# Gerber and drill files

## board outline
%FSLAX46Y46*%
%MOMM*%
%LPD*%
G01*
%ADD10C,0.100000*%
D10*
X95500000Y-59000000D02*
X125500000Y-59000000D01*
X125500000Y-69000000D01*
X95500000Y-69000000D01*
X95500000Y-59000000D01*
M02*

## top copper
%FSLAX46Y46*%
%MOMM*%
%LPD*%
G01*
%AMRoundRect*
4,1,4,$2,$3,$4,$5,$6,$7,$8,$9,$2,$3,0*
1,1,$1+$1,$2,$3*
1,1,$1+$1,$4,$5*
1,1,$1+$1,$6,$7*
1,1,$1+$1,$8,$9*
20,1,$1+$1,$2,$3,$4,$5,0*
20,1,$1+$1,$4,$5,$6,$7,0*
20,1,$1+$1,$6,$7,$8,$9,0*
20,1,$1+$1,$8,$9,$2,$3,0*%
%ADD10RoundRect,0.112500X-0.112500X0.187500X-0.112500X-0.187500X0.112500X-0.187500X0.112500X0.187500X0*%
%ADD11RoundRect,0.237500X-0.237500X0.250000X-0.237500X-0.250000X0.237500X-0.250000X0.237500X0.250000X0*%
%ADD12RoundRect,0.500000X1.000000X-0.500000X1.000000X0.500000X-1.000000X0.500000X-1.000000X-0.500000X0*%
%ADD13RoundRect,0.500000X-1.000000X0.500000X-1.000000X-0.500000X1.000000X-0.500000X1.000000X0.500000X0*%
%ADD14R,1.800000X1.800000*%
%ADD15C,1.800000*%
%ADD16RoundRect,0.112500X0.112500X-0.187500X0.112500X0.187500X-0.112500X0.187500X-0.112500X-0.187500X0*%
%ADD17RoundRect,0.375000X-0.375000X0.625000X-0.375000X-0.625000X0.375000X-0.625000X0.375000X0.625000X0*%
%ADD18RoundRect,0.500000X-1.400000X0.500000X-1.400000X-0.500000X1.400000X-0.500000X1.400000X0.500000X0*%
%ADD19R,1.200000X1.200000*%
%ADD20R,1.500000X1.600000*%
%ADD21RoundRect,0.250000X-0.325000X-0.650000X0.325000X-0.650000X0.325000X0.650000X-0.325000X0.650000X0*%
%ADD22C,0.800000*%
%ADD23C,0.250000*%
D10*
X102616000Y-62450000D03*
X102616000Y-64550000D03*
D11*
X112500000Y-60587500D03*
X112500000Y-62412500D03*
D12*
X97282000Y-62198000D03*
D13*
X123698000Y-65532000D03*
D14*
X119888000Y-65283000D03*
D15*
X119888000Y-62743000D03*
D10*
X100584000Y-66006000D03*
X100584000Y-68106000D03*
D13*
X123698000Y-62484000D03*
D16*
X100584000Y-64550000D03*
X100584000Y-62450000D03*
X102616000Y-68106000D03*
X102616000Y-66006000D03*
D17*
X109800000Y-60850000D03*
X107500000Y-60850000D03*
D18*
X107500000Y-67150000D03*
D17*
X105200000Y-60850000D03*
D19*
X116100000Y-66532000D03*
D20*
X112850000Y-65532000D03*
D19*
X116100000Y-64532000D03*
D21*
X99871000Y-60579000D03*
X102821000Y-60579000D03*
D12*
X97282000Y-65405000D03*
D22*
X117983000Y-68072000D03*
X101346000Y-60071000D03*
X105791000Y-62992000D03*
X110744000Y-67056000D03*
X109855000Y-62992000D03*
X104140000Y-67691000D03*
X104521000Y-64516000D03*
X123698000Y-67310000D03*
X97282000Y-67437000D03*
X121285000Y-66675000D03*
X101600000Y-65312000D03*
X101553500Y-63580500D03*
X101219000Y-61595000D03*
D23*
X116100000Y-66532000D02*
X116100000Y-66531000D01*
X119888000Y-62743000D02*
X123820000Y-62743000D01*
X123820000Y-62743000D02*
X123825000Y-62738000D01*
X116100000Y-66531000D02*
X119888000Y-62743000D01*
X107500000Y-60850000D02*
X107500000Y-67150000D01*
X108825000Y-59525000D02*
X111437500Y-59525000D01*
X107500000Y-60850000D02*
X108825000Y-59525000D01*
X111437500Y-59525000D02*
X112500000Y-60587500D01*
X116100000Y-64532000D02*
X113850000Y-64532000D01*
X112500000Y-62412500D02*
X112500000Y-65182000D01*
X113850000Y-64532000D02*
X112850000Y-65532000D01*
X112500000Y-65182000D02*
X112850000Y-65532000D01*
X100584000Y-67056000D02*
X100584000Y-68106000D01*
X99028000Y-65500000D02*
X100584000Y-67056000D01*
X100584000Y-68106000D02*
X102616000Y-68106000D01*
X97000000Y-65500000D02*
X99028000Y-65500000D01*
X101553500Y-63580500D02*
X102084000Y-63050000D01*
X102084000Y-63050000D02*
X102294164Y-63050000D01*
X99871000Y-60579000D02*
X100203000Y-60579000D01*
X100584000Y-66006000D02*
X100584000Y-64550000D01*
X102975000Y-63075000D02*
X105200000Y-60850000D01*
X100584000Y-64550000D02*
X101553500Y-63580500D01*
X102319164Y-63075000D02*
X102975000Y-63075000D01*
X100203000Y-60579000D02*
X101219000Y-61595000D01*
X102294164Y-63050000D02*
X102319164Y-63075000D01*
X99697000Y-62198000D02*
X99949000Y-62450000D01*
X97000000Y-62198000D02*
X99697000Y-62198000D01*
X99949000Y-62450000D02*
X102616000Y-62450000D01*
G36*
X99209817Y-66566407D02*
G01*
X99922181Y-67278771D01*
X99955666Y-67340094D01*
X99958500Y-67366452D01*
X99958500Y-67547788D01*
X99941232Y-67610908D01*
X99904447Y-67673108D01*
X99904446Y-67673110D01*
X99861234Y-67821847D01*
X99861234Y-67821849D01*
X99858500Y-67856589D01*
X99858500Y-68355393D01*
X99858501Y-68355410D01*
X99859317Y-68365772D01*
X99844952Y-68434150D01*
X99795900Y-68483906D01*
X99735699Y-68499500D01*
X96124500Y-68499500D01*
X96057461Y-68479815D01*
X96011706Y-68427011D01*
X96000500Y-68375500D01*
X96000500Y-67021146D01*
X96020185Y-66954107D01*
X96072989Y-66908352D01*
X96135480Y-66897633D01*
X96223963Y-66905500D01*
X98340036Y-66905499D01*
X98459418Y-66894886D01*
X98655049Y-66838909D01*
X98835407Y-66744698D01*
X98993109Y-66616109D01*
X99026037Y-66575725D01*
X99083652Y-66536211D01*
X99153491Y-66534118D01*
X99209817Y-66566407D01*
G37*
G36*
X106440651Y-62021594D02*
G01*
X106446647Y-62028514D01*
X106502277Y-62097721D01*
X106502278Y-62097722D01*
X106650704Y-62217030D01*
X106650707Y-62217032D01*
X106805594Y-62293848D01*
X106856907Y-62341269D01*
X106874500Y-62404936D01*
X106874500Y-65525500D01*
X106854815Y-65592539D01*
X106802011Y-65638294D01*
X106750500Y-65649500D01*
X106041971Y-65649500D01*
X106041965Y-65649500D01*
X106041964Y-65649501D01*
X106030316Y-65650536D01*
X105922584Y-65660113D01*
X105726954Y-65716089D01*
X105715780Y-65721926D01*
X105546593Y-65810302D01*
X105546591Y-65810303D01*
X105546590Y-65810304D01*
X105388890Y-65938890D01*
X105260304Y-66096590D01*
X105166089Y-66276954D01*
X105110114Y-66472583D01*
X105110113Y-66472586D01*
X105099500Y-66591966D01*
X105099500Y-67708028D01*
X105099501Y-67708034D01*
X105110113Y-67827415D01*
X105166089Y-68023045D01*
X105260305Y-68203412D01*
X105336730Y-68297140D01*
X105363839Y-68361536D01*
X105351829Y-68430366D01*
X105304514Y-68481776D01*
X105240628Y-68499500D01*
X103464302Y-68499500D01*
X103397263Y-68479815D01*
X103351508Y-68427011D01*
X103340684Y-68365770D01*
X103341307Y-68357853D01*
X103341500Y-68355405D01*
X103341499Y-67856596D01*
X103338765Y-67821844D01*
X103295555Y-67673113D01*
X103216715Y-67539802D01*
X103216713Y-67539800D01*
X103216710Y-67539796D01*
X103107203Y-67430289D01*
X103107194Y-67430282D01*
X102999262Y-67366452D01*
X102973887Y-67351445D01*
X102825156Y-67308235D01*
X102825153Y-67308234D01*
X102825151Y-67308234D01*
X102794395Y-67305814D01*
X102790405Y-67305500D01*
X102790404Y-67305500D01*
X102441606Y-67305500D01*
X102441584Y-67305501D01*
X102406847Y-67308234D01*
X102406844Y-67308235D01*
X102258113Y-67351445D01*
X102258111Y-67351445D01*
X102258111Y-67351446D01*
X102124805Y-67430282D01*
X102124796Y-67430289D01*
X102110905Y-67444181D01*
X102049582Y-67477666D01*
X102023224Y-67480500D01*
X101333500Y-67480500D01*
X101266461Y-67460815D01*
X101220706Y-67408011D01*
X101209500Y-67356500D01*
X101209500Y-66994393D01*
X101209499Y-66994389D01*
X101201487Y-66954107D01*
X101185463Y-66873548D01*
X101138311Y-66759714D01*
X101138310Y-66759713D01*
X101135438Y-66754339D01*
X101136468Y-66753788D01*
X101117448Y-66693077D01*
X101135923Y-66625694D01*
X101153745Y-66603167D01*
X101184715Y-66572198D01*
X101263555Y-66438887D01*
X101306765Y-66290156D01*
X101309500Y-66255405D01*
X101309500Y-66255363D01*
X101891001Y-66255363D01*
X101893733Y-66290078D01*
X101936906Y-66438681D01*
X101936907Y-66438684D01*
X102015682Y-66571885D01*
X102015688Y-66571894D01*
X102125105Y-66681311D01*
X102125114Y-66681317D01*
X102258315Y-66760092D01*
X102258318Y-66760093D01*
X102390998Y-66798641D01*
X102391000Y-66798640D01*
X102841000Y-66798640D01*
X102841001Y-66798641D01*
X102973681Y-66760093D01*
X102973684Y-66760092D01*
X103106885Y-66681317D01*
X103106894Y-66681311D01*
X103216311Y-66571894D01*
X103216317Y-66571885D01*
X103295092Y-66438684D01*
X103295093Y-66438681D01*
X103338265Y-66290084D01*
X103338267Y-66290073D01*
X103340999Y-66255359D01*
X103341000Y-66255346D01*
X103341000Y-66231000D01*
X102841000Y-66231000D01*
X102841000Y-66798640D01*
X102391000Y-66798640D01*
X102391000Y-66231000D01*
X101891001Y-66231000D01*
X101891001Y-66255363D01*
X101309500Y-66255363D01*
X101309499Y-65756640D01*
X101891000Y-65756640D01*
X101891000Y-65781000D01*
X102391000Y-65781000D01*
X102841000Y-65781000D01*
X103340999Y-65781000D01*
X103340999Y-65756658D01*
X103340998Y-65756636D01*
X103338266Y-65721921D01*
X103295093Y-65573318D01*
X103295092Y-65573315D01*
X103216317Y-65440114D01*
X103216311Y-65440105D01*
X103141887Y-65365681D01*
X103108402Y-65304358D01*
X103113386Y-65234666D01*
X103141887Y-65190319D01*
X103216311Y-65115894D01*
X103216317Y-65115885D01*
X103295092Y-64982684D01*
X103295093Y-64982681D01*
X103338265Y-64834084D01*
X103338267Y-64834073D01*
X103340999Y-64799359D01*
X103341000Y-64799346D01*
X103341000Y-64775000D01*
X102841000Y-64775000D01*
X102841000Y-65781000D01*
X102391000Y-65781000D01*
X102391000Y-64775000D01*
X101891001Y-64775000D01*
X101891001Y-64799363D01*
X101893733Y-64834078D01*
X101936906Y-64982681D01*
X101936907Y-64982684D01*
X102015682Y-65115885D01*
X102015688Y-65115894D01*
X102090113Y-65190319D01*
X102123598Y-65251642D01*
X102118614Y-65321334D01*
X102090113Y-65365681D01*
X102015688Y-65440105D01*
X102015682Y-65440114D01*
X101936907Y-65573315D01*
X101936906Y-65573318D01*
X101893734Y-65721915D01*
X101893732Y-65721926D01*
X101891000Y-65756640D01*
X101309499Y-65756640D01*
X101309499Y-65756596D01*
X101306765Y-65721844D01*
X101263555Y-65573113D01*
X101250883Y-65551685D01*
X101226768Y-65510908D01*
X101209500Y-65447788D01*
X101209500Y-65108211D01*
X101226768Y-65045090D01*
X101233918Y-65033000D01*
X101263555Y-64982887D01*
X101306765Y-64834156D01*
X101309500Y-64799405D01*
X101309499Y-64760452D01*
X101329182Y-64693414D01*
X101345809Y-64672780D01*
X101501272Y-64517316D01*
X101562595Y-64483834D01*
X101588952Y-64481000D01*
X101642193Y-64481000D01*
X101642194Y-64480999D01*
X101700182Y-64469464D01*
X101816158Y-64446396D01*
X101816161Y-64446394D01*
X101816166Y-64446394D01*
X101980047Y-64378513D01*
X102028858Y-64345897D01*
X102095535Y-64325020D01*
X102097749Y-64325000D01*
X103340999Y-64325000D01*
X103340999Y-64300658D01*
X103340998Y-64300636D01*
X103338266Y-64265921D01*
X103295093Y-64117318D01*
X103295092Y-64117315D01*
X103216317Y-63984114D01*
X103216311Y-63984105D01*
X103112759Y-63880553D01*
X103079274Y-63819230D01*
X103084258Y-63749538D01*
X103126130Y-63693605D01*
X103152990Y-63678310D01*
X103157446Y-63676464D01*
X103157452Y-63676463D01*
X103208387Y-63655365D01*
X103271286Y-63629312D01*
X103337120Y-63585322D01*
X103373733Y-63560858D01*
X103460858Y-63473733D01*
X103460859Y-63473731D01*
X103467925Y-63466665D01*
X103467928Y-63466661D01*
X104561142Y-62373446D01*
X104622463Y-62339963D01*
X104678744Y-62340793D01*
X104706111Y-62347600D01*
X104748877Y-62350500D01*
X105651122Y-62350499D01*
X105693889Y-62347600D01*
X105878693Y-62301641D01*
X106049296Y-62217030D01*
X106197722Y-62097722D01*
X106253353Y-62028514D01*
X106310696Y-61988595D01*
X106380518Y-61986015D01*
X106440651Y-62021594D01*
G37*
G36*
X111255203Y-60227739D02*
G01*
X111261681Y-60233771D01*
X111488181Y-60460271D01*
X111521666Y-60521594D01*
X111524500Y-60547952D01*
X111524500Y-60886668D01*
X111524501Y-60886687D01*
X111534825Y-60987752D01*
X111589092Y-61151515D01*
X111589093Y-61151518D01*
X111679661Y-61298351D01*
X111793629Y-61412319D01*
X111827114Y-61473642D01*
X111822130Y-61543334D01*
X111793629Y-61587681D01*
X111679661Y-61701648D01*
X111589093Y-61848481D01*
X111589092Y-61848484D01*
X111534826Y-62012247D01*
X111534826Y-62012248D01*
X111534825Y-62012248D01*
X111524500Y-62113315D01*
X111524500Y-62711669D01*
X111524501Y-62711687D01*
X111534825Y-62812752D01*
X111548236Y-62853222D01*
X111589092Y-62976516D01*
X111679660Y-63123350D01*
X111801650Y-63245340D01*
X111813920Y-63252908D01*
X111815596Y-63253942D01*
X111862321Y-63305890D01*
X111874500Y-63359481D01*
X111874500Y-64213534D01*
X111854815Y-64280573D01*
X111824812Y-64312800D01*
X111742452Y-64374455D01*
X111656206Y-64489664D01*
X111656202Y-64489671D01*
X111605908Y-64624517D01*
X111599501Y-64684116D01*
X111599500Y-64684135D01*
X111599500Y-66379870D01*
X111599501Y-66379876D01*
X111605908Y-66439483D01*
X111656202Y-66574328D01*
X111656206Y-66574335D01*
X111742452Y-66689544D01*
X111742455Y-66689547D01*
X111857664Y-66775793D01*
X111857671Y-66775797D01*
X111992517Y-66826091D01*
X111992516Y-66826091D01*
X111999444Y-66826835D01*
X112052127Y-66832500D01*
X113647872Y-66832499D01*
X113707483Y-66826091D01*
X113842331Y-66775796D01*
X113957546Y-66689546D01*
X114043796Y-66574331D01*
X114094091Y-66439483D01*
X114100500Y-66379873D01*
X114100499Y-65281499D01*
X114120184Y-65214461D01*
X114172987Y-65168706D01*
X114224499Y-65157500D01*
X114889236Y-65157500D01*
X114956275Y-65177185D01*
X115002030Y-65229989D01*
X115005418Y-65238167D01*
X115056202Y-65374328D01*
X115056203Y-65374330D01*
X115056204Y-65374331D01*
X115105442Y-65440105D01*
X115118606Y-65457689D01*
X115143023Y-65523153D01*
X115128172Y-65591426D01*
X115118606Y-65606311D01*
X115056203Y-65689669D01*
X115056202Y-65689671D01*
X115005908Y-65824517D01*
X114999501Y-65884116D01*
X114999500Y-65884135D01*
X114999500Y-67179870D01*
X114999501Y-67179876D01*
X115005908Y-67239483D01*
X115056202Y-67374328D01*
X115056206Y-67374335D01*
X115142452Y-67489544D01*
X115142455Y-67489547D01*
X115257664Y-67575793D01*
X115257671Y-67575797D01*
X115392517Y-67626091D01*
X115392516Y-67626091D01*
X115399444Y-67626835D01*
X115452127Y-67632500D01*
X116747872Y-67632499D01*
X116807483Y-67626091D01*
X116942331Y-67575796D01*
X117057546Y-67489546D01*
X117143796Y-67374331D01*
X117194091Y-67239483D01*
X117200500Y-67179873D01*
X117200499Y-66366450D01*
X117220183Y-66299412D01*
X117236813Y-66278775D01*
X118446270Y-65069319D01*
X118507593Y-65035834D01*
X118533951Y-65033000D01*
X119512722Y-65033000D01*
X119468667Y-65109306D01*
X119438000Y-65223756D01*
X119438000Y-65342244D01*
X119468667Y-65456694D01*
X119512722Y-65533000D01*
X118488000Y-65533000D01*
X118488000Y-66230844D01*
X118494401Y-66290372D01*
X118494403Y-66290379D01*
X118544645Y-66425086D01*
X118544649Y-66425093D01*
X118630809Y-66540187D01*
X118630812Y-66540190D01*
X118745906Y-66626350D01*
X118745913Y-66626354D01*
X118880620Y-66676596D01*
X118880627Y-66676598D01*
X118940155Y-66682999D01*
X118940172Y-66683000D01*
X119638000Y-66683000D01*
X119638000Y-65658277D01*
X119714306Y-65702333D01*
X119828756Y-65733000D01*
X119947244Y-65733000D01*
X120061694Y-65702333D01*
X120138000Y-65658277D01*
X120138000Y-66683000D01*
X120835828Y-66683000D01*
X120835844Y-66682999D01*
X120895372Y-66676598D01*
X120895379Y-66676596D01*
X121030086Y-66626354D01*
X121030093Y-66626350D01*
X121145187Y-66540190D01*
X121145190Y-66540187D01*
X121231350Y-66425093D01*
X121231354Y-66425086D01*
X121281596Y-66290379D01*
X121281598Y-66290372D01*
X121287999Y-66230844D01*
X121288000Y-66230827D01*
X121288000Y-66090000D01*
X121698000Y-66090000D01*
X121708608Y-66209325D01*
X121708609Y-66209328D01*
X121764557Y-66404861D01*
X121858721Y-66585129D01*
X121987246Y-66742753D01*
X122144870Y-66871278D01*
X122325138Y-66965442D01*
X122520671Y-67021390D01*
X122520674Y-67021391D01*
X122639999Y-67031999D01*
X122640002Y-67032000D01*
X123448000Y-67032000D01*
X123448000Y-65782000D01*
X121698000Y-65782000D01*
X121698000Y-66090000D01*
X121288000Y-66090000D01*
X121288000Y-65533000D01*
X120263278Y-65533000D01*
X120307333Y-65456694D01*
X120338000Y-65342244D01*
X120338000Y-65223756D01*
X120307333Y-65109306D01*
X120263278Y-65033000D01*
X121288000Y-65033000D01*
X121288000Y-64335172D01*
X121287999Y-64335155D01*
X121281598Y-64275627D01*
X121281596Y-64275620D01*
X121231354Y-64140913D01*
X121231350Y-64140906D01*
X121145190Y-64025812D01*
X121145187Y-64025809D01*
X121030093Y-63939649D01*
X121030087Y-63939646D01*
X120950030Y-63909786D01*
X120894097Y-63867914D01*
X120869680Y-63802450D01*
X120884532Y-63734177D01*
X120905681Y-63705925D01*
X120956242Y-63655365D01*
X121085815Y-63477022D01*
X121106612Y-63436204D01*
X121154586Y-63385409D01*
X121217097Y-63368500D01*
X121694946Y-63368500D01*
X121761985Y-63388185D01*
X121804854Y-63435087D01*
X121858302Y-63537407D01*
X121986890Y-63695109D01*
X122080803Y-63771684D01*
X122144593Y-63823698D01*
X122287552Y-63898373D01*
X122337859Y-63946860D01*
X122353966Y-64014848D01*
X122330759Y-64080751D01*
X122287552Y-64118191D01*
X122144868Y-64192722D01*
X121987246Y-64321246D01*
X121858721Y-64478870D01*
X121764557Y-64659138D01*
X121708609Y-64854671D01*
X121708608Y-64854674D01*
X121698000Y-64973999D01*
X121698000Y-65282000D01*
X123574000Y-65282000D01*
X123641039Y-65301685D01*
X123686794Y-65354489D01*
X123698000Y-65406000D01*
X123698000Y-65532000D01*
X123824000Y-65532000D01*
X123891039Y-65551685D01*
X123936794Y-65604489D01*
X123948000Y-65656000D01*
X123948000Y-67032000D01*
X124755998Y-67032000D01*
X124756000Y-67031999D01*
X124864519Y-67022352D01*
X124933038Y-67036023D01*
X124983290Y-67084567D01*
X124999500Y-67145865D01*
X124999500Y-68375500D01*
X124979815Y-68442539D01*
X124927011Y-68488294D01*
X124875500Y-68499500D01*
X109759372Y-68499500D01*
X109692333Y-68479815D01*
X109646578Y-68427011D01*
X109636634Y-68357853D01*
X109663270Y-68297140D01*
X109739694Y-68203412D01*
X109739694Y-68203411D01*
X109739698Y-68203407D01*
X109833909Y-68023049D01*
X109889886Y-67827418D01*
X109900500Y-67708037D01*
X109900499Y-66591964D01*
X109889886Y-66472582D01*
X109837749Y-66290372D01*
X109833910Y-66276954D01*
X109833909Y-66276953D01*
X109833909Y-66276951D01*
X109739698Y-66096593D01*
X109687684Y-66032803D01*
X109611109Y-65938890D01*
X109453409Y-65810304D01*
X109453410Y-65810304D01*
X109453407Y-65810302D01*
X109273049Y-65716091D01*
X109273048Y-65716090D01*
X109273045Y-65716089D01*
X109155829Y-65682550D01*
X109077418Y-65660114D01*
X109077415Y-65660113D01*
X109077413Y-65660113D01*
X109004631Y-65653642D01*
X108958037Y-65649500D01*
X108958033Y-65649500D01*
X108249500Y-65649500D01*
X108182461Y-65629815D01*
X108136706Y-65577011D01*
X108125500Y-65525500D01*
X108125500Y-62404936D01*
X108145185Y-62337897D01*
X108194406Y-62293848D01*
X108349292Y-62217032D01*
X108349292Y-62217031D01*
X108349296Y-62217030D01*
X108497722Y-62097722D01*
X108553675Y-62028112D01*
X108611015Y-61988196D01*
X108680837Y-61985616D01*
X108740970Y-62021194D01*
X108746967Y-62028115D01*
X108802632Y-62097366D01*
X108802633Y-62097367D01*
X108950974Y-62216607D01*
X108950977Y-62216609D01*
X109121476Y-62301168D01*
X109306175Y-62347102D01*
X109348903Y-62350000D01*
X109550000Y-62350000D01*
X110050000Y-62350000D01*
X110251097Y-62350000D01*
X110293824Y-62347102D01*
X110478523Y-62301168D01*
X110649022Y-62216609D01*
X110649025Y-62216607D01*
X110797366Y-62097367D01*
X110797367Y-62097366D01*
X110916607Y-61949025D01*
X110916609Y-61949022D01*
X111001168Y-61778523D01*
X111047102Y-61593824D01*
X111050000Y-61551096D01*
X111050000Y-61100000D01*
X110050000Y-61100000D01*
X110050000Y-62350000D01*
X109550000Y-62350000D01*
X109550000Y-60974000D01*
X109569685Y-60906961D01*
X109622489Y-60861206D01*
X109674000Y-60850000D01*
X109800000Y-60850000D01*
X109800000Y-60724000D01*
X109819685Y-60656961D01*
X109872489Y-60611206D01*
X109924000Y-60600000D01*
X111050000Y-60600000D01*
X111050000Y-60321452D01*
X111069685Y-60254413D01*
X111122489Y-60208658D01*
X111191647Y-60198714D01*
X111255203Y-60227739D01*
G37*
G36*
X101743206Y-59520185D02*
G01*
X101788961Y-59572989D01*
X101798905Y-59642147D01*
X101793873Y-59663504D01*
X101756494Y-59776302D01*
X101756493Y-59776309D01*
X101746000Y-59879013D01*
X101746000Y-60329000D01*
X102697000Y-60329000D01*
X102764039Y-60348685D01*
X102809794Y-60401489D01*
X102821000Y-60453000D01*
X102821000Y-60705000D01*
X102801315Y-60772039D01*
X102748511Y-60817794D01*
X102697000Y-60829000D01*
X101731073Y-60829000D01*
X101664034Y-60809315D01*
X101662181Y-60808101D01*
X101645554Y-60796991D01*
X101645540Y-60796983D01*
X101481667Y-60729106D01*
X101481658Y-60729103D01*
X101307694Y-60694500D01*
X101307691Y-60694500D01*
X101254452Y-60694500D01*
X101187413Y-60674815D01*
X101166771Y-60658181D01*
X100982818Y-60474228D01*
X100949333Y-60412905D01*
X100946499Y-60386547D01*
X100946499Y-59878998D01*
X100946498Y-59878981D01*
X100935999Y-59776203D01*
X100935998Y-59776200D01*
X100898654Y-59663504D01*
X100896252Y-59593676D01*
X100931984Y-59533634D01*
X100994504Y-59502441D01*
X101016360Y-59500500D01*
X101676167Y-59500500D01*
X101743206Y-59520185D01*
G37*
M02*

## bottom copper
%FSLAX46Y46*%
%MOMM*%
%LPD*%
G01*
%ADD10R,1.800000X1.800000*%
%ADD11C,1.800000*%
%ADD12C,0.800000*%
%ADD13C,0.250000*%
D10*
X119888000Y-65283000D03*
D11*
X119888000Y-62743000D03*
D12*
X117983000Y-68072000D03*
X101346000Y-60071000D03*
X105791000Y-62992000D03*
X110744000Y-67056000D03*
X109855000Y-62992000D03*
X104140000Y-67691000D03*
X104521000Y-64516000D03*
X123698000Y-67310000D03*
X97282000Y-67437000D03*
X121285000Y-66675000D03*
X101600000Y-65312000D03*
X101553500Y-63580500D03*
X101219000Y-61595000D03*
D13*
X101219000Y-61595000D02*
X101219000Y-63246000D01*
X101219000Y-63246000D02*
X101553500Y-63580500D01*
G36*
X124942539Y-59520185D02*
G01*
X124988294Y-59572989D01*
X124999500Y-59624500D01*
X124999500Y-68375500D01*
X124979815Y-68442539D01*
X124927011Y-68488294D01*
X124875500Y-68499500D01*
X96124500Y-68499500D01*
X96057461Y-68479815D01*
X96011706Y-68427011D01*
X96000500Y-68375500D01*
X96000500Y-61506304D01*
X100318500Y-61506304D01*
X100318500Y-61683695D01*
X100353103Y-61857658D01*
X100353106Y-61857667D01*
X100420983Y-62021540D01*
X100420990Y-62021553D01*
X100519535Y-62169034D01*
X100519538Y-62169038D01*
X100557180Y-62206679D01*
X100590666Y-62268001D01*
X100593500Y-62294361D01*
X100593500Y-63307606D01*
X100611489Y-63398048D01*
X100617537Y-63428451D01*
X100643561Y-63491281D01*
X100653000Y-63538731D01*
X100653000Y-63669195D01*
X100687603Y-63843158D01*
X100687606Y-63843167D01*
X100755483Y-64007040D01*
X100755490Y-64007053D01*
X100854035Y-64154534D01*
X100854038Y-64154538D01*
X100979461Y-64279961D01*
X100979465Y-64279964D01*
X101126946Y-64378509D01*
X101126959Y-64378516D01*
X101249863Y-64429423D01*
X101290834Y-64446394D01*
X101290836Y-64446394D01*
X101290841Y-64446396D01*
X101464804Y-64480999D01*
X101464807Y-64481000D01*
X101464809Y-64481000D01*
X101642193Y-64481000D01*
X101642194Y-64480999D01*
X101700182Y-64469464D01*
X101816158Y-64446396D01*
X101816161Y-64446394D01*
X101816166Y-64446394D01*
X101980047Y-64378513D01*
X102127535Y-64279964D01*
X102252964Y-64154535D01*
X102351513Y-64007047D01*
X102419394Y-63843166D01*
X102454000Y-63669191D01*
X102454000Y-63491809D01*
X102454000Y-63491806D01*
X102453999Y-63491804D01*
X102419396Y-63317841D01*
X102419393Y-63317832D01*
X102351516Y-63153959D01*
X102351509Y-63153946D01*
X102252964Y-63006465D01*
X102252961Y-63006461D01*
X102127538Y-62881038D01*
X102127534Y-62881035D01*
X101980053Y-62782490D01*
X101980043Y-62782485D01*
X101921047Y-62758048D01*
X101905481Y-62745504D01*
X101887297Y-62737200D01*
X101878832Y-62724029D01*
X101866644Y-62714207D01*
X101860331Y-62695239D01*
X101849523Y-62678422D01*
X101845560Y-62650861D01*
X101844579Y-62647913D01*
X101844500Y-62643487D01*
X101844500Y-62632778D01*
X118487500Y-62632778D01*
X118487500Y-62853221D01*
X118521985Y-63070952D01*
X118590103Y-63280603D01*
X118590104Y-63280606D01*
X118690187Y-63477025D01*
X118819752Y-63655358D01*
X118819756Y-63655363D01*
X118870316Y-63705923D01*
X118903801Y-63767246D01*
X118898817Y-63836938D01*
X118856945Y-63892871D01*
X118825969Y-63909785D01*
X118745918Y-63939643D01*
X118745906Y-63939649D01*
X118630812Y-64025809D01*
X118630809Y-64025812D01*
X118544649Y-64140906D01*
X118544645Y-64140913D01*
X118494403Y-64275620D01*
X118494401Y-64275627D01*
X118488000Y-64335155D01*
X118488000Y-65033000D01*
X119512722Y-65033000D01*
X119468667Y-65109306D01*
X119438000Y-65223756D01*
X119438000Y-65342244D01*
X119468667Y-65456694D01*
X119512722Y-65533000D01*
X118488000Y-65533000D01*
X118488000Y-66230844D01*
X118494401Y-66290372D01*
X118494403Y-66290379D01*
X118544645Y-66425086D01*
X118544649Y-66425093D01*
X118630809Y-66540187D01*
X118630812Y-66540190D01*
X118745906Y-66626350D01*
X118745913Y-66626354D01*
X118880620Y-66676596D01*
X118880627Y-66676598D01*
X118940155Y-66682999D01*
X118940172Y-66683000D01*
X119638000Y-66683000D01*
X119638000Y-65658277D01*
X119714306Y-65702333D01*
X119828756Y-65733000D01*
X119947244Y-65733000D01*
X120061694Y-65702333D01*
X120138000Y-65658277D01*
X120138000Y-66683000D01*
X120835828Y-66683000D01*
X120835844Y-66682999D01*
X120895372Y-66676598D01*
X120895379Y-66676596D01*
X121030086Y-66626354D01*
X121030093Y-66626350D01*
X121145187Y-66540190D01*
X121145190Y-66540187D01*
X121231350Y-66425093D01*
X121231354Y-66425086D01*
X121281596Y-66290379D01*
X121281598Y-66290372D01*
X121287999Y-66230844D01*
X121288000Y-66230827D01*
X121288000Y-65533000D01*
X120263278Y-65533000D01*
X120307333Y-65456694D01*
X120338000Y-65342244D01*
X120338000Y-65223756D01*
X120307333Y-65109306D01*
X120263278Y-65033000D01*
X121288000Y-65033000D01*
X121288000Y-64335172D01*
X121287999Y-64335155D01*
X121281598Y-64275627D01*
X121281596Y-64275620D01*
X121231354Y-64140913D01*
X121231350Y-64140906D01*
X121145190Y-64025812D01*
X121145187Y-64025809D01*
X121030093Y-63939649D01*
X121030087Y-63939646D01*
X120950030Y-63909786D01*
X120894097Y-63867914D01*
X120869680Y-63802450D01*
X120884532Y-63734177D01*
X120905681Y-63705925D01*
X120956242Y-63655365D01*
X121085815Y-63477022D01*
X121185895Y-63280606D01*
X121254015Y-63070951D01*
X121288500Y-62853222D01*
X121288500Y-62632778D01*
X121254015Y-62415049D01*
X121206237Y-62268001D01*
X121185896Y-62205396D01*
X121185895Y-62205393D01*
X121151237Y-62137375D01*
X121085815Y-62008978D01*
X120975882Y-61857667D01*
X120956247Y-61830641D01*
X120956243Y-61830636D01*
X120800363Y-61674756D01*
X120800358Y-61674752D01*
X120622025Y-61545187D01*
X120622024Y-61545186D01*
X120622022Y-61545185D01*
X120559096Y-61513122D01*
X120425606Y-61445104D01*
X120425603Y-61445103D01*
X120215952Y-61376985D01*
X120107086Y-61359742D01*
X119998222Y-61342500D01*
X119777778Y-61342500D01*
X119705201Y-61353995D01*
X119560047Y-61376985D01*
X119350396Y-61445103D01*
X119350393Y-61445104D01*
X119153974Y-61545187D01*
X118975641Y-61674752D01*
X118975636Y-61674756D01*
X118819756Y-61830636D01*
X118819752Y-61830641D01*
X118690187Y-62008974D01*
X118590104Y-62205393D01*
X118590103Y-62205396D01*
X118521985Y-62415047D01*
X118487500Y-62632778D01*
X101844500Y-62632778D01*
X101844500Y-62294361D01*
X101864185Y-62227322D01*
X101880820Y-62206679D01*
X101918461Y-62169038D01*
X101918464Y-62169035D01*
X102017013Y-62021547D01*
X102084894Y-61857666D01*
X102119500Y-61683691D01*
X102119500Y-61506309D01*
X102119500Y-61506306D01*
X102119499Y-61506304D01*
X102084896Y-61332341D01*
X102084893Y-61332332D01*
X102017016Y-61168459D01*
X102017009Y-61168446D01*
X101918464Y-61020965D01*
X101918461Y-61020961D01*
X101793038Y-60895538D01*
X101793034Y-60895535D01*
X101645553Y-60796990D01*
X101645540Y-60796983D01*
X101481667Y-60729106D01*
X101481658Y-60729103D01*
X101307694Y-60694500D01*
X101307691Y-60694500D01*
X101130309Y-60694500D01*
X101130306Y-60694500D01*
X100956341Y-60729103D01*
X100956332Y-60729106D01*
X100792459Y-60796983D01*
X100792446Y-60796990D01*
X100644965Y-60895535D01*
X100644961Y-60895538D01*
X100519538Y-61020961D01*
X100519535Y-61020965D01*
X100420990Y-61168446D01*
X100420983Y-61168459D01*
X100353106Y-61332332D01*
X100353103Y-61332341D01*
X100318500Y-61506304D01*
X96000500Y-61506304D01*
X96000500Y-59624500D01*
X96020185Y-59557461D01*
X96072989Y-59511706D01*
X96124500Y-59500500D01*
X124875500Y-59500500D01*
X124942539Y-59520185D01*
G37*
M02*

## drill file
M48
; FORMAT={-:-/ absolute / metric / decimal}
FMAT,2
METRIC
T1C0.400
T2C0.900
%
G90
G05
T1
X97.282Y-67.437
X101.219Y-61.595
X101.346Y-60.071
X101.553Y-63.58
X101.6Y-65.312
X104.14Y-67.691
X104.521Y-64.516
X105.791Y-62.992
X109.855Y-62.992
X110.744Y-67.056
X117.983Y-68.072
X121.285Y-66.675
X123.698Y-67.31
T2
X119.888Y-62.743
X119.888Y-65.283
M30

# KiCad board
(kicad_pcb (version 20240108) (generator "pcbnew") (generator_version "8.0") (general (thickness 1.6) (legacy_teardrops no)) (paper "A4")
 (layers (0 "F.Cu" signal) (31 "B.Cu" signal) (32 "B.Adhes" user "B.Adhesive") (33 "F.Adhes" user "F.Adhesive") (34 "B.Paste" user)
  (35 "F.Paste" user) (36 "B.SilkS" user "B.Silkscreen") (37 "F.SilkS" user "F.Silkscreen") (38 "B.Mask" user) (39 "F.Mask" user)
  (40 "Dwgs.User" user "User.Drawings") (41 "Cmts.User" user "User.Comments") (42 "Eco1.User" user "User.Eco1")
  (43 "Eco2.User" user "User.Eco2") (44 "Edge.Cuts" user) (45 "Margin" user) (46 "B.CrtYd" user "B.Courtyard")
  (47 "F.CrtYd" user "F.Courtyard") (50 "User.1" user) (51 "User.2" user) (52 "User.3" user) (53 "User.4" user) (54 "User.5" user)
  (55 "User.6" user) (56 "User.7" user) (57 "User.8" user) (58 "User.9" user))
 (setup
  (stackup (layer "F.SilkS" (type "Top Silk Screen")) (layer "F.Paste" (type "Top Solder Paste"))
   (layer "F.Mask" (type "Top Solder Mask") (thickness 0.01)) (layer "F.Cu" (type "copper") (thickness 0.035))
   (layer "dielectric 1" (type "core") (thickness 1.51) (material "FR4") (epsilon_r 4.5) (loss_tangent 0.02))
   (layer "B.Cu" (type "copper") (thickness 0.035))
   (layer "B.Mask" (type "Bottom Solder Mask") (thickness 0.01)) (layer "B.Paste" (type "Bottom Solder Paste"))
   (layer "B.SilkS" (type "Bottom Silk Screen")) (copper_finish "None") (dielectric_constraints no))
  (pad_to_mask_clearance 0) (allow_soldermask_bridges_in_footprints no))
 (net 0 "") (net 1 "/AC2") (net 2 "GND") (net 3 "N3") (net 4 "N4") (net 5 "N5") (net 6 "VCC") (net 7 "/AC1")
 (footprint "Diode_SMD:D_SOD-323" (layer "F.Cu") (at 102.616 63.5 -90)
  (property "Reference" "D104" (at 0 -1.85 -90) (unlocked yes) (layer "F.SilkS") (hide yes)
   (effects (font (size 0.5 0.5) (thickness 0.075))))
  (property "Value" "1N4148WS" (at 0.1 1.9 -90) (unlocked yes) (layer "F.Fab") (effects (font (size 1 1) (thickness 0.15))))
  (pad "1" smd roundrect (at -1.05 0 270) (size 0.6 0.45) (layers "F.Cu" "F.Paste" "F.Mask") (roundrect_rratio 0.25) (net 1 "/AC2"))
  (pad "2" smd roundrect (at 1.05 0 270) (size 0.6 0.45) (layers "F.Cu" "F.Paste" "F.Mask") (roundrect_rratio 0.25) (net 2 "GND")))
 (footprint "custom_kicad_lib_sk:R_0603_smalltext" (layer "F.Cu") (at 112.5 61.5 -90)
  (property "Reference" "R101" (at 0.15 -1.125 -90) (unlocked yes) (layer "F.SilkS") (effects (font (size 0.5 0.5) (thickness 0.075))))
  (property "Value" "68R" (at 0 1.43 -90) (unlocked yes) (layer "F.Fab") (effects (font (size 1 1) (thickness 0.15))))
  (pad "1" smd roundrect (at -0.9125 0 270) (size 0.975 0.95) (layers "F.Cu" "F.Paste" "F.Mask") (roundrect_rratio 0.25) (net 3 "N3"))
  (pad "2" smd roundrect (at 0.9125 0 270) (size 0.975 0.95) (layers "F.Cu" "F.Paste" "F.Mask") (roundrect_rratio 0.25) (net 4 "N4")))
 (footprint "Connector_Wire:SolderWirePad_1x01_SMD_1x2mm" (layer "F.Cu") (at 97.282 62.198 90)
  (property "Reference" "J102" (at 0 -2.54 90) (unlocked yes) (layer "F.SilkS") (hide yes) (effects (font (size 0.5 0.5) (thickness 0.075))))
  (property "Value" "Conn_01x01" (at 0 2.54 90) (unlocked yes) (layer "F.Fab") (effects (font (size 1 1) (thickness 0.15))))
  (pad "1" smd roundrect (at 0 0 90) (size 2 3) (layers "F.Cu" "F.Paste" "F.Mask") (roundrect_rratio 0.25) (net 1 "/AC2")))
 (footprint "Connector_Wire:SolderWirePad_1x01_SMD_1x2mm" (layer "F.Cu") (at 123.698 65.532 -90)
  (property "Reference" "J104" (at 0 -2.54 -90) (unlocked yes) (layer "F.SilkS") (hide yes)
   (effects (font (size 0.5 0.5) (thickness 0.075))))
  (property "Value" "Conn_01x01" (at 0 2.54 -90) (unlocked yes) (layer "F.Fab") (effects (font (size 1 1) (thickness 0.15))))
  (pad "1" smd roundrect (at 0 0 270) (size 2 3) (layers "F.Cu" "F.Paste" "F.Mask") (roundrect_rratio 0.25) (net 2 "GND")))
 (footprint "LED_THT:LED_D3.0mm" (layer "F.Cu") (at 119.888 65.283 90)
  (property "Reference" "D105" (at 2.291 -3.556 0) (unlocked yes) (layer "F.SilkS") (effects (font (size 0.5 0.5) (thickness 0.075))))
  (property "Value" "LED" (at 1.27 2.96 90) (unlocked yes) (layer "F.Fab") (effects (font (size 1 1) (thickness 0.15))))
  (pad "1" thru_hole rect (at 0 0 90) (size 1.8 1.8) (drill 0.9) (layers "*.Cu" "*.Mask") (remove_unused_layers no) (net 2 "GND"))
  (pad "2" thru_hole circle (at 2.54 0 90) (size 1.8 1.8) (drill 0.9) (layers "*.Cu" "*.Mask") (remove_unused_layers no) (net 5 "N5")))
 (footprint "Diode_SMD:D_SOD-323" (layer "F.Cu") (at 100.584 67.056 -90)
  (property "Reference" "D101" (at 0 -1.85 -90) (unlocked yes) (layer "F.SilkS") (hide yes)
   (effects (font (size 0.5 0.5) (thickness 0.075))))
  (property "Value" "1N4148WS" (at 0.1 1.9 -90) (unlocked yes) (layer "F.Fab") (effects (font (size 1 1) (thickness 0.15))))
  (pad "1" smd roundrect (at -1.05 0 270) (size 0.6 0.45) (layers "F.Cu" "F.Paste" "F.Mask") (roundrect_rratio 0.25) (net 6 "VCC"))
  (pad "2" smd roundrect (at 1.05 0 270) (size 0.6 0.45) (layers "F.Cu" "F.Paste" "F.Mask") (roundrect_rratio 0.25) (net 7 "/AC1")))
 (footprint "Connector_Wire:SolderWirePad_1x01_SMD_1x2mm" (layer "F.Cu") (at 123.698 62.484 -90)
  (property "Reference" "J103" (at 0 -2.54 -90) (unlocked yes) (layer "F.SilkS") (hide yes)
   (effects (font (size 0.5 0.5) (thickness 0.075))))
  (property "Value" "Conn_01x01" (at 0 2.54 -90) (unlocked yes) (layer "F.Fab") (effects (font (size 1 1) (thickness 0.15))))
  (pad "1" smd roundrect (at 0 0 270) (size 2 3) (layers "F.Cu" "F.Paste" "F.Mask") (roundrect_rratio 0.25) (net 5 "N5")))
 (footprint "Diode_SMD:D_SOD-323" (layer "F.Cu") (at 100.584 63.5 90)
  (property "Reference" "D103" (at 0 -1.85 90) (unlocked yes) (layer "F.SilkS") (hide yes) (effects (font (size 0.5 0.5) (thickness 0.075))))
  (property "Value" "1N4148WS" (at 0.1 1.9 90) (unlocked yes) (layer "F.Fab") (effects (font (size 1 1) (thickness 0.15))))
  (pad "1" smd roundrect (at -1.05 0 90) (size 0.6 0.45) (layers "F.Cu" "F.Paste" "F.Mask") (roundrect_rratio 0.25) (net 6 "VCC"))
  (pad "2" smd roundrect (at 1.05 0 90) (size 0.6 0.45) (layers "F.Cu" "F.Paste" "F.Mask") (roundrect_rratio 0.25) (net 1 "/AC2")))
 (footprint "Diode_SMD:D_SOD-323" (layer "F.Cu") (at 102.616 67.056 90)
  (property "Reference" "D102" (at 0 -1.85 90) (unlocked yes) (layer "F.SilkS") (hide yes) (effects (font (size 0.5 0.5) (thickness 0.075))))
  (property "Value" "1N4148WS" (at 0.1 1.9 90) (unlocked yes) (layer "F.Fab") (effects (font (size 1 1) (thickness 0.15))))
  (pad "1" smd roundrect (at -1.05 0 90) (size 0.6 0.45) (layers "F.Cu" "F.Paste" "F.Mask") (roundrect_rratio 0.25) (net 7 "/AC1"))
  (pad "2" smd roundrect (at 1.05 0 90) (size 0.6 0.45) (layers "F.Cu" "F.Paste" "F.Mask") (roundrect_rratio 0.25) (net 2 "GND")))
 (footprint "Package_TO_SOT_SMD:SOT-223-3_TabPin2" (layer "F.Cu") (at 107.5 64 -90)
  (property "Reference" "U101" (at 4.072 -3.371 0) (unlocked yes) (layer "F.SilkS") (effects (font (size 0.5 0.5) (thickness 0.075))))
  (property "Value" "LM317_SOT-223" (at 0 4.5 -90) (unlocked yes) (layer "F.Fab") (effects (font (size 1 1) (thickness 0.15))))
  (pad "1" smd roundrect (at -3.15 -2.3 270) (size 2 1.5) (layers "F.Cu" "F.Paste" "F.Mask") (roundrect_rratio 0.25) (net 2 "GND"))
  (pad "2" smd roundrect (at -3.15 0 270) (size 2 1.5) (layers "F.Cu" "F.Paste" "F.Mask") (roundrect_rratio 0.25) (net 3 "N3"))
  (pad "2" smd roundrect (at 3.15 0 270) (size 2 3.8) (layers "F.Cu" "F.Paste" "F.Mask") (roundrect_rratio 0.25) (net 3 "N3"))
  (pad "3" smd roundrect (at -3.15 2.3 270) (size 2 1.5) (layers "F.Cu" "F.Paste" "F.Mask") (roundrect_rratio 0.25) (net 6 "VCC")))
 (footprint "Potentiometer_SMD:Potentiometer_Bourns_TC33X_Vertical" (layer "F.Cu") (at 114.3 65.532 180)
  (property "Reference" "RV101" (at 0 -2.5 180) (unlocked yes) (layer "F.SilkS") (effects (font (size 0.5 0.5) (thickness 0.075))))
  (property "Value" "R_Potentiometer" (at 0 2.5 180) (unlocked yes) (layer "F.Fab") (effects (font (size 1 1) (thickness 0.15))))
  (pad "1" smd rect (at -1.8 -1 180) (size 1.2 1.2) (layers "F.Cu" "F.Paste" "F.Mask") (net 5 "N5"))
  (pad "2" smd rect (at 1.45 0 180) (size 1.5 1.6) (layers "F.Cu" "F.Paste" "F.Mask") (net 4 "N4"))
  (pad "3" smd rect (at -1.8 1 180) (size 1.2 1.2) (layers "F.Cu" "F.Paste" "F.Mask") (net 4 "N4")))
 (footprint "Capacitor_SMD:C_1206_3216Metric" (layer "F.Cu") (at 101.346 60.579)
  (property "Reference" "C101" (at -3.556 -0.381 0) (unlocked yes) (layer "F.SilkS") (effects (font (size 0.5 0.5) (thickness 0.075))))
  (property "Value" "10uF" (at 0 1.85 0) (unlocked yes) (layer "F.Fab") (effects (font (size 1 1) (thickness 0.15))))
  (pad "1" smd roundrect (at -1.475 0) (size 1.15 1.8) (layers "F.Cu" "F.Paste" "F.Mask") (roundrect_rratio 0.217391) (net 6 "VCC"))
  (pad "2" smd roundrect (at 1.475 0) (size 1.15 1.8) (layers "F.Cu" "F.Paste" "F.Mask") (roundrect_rratio 0.217391) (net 2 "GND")))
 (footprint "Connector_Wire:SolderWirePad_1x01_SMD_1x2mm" (layer "F.Cu") (at 97.282 65.405 90)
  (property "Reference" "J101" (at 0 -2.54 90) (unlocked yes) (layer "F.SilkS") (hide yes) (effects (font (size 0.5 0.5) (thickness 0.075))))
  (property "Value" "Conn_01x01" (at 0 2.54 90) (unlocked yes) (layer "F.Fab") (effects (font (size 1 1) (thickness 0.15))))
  (pad "1" smd roundrect (at 0 0 90) (size 2 3) (layers "F.Cu" "F.Paste" "F.Mask") (roundrect_rratio 0.25) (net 7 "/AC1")))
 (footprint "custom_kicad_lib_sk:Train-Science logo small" (layer "B.Cu") (at 101.6 64.008 90)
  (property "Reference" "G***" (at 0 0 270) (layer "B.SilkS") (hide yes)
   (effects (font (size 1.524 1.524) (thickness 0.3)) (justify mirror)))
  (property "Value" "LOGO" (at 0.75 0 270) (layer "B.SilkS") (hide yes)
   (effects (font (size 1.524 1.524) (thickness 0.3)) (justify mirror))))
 (gr_rect (start 95.5 59) (end 125.5 69) (stroke (width 0.1) (type default)) (fill none) (layer "Edge.Cuts"))
 (via (at 117.983 68.072) (size 0.8) (drill 0.4) (layers "F.Cu" "B.Cu") (free yes) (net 2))
 (via (at 101.346 60.071) (size 0.8) (drill 0.4) (layers "F.Cu" "B.Cu") (free yes) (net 2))
 (via (at 105.791 62.992) (size 0.8) (drill 0.4) (layers "F.Cu" "B.Cu") (free yes) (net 2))
 (via (at 110.744 67.056) (size 0.8) (drill 0.4) (layers "F.Cu" "B.Cu") (free yes) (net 2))
 (via (at 109.855 62.992) (size 0.8) (drill 0.4) (layers "F.Cu" "B.Cu") (free yes) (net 2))
 (via (at 104.14 67.691) (size 0.8) (drill 0.4) (layers "F.Cu" "B.Cu") (free yes) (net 2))
 (via (at 104.521 64.516) (size 0.8) (drill 0.4) (layers "F.Cu" "B.Cu") (free yes) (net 2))
 (via (at 123.698 67.31) (size 0.8) (drill 0.4) (layers "F.Cu" "B.Cu") (free yes) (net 2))
 (via (at 97.282 67.437) (size 0.8) (drill 0.4) (layers "F.Cu" "B.Cu") (free yes) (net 2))
 (via (at 121.285 66.675) (size 0.8) (drill 0.4) (layers "F.Cu" "B.Cu") (free yes) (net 2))
 (via (at 101.6 65.312) (size 0.8) (drill 0.4) (layers "F.Cu" "B.Cu") (free yes) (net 2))
 (segment (start 116.1 66.532) (end 116.1 66.531) (width 0.25) (layer "F.Cu") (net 5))
 (segment (start 119.888 62.743) (end 123.82 62.743) (width 0.25) (layer "F.Cu") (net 5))
 (segment (start 123.82 62.743) (end 123.825 62.738) (width 0.25) (layer "F.Cu") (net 5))
 (segment (start 116.1 66.531) (end 119.888 62.743) (width 0.25) (layer "F.Cu") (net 5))
 (segment (start 107.5 60.85) (end 107.5 67.15) (width 0.25) (layer "F.Cu") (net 3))
 (segment (start 108.825 59.525) (end 111.4375 59.525) (width 0.25) (layer "F.Cu") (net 3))
 (segment (start 107.5 60.85) (end 108.825 59.525) (width 0.25) (layer "F.Cu") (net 3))
 (segment (start 111.4375 59.525) (end 112.5 60.5875) (width 0.25) (layer "F.Cu") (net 3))
 (segment (start 116.1 64.532) (end 113.85 64.532) (width 0.25) (layer "F.Cu") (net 4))
 (segment (start 112.5 62.4125) (end 112.5 65.182) (width 0.25) (layer "F.Cu") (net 4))
 (segment (start 113.85 64.532) (end 112.85 65.532) (width 0.25) (layer "F.Cu") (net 4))
 (segment (start 112.5 65.182) (end 112.85 65.532) (width 0.25) (layer "F.Cu") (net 4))
 (segment (start 100.584 67.056) (end 100.584 68.106) (width 0.25) (layer "F.Cu") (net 7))
 (segment (start 99.028 65.5) (end 100.584 67.056) (width 0.25) (layer "F.Cu") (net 7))
 (segment (start 100.584 68.106) (end 102.616 68.106) (width 0.25) (layer "F.Cu") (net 7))
 (segment (start 97 65.5) (end 99.028 65.5) (width 0.25) (layer "F.Cu") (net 7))
 (segment (start 101.5535 63.5805) (end 102.084 63.05) (width 0.25) (layer "F.Cu") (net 6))
 (segment (start 102.084 63.05) (end 102.294164 63.05) (width 0.25) (layer "F.Cu") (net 6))
 (segment (start 99.871 60.579) (end 100.203 60.579) (width 0.25) (layer "F.Cu") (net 6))
 (segment (start 100.584 66.006) (end 100.584 64.55) (width 0.25) (layer "F.Cu") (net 6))
 (segment (start 102.975 63.075) (end 105.2 60.85) (width 0.25) (layer "F.Cu") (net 6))
 (segment (start 100.584 64.55) (end 101.5535 63.5805) (width 0.25) (layer "F.Cu") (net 6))
 (segment (start 102.319164 63.075) (end 102.975 63.075) (width 0.25) (layer "F.Cu") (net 6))
 (segment (start 100.203 60.579) (end 101.219 61.595) (width 0.25) (layer "F.Cu") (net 6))
 (segment (start 102.294164 63.05) (end 102.319164 63.075) (width 0.25) (layer "F.Cu") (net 6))
 (via (at 101.5535 63.5805) (size 0.8) (drill 0.4) (layers "F.Cu" "B.Cu") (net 6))
 (via (at 101.219 61.595) (size 0.8) (drill 0.4) (layers "F.Cu" "B.Cu") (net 6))
 (segment (start 101.219 61.595) (end 101.219 63.246) (width 0.25) (layer "B.Cu") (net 6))
 (segment (start 101.219 63.246) (end 101.5535 63.5805) (width 0.25) (layer "B.Cu") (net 6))
 (segment (start 99.697 62.198) (end 99.949 62.45) (width 0.25) (layer "F.Cu") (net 1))
 (segment (start 97 62.198) (end 99.697 62.198) (width 0.25) (layer "F.Cu") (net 1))
 (segment (start 99.949 62.45) (end 102.616 62.45) (width 0.25) (layer "F.Cu") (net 1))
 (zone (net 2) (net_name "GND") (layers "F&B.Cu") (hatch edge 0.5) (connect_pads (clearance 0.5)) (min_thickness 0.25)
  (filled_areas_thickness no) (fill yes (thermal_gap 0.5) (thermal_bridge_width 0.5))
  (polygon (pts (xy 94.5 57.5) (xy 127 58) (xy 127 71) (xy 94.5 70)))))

